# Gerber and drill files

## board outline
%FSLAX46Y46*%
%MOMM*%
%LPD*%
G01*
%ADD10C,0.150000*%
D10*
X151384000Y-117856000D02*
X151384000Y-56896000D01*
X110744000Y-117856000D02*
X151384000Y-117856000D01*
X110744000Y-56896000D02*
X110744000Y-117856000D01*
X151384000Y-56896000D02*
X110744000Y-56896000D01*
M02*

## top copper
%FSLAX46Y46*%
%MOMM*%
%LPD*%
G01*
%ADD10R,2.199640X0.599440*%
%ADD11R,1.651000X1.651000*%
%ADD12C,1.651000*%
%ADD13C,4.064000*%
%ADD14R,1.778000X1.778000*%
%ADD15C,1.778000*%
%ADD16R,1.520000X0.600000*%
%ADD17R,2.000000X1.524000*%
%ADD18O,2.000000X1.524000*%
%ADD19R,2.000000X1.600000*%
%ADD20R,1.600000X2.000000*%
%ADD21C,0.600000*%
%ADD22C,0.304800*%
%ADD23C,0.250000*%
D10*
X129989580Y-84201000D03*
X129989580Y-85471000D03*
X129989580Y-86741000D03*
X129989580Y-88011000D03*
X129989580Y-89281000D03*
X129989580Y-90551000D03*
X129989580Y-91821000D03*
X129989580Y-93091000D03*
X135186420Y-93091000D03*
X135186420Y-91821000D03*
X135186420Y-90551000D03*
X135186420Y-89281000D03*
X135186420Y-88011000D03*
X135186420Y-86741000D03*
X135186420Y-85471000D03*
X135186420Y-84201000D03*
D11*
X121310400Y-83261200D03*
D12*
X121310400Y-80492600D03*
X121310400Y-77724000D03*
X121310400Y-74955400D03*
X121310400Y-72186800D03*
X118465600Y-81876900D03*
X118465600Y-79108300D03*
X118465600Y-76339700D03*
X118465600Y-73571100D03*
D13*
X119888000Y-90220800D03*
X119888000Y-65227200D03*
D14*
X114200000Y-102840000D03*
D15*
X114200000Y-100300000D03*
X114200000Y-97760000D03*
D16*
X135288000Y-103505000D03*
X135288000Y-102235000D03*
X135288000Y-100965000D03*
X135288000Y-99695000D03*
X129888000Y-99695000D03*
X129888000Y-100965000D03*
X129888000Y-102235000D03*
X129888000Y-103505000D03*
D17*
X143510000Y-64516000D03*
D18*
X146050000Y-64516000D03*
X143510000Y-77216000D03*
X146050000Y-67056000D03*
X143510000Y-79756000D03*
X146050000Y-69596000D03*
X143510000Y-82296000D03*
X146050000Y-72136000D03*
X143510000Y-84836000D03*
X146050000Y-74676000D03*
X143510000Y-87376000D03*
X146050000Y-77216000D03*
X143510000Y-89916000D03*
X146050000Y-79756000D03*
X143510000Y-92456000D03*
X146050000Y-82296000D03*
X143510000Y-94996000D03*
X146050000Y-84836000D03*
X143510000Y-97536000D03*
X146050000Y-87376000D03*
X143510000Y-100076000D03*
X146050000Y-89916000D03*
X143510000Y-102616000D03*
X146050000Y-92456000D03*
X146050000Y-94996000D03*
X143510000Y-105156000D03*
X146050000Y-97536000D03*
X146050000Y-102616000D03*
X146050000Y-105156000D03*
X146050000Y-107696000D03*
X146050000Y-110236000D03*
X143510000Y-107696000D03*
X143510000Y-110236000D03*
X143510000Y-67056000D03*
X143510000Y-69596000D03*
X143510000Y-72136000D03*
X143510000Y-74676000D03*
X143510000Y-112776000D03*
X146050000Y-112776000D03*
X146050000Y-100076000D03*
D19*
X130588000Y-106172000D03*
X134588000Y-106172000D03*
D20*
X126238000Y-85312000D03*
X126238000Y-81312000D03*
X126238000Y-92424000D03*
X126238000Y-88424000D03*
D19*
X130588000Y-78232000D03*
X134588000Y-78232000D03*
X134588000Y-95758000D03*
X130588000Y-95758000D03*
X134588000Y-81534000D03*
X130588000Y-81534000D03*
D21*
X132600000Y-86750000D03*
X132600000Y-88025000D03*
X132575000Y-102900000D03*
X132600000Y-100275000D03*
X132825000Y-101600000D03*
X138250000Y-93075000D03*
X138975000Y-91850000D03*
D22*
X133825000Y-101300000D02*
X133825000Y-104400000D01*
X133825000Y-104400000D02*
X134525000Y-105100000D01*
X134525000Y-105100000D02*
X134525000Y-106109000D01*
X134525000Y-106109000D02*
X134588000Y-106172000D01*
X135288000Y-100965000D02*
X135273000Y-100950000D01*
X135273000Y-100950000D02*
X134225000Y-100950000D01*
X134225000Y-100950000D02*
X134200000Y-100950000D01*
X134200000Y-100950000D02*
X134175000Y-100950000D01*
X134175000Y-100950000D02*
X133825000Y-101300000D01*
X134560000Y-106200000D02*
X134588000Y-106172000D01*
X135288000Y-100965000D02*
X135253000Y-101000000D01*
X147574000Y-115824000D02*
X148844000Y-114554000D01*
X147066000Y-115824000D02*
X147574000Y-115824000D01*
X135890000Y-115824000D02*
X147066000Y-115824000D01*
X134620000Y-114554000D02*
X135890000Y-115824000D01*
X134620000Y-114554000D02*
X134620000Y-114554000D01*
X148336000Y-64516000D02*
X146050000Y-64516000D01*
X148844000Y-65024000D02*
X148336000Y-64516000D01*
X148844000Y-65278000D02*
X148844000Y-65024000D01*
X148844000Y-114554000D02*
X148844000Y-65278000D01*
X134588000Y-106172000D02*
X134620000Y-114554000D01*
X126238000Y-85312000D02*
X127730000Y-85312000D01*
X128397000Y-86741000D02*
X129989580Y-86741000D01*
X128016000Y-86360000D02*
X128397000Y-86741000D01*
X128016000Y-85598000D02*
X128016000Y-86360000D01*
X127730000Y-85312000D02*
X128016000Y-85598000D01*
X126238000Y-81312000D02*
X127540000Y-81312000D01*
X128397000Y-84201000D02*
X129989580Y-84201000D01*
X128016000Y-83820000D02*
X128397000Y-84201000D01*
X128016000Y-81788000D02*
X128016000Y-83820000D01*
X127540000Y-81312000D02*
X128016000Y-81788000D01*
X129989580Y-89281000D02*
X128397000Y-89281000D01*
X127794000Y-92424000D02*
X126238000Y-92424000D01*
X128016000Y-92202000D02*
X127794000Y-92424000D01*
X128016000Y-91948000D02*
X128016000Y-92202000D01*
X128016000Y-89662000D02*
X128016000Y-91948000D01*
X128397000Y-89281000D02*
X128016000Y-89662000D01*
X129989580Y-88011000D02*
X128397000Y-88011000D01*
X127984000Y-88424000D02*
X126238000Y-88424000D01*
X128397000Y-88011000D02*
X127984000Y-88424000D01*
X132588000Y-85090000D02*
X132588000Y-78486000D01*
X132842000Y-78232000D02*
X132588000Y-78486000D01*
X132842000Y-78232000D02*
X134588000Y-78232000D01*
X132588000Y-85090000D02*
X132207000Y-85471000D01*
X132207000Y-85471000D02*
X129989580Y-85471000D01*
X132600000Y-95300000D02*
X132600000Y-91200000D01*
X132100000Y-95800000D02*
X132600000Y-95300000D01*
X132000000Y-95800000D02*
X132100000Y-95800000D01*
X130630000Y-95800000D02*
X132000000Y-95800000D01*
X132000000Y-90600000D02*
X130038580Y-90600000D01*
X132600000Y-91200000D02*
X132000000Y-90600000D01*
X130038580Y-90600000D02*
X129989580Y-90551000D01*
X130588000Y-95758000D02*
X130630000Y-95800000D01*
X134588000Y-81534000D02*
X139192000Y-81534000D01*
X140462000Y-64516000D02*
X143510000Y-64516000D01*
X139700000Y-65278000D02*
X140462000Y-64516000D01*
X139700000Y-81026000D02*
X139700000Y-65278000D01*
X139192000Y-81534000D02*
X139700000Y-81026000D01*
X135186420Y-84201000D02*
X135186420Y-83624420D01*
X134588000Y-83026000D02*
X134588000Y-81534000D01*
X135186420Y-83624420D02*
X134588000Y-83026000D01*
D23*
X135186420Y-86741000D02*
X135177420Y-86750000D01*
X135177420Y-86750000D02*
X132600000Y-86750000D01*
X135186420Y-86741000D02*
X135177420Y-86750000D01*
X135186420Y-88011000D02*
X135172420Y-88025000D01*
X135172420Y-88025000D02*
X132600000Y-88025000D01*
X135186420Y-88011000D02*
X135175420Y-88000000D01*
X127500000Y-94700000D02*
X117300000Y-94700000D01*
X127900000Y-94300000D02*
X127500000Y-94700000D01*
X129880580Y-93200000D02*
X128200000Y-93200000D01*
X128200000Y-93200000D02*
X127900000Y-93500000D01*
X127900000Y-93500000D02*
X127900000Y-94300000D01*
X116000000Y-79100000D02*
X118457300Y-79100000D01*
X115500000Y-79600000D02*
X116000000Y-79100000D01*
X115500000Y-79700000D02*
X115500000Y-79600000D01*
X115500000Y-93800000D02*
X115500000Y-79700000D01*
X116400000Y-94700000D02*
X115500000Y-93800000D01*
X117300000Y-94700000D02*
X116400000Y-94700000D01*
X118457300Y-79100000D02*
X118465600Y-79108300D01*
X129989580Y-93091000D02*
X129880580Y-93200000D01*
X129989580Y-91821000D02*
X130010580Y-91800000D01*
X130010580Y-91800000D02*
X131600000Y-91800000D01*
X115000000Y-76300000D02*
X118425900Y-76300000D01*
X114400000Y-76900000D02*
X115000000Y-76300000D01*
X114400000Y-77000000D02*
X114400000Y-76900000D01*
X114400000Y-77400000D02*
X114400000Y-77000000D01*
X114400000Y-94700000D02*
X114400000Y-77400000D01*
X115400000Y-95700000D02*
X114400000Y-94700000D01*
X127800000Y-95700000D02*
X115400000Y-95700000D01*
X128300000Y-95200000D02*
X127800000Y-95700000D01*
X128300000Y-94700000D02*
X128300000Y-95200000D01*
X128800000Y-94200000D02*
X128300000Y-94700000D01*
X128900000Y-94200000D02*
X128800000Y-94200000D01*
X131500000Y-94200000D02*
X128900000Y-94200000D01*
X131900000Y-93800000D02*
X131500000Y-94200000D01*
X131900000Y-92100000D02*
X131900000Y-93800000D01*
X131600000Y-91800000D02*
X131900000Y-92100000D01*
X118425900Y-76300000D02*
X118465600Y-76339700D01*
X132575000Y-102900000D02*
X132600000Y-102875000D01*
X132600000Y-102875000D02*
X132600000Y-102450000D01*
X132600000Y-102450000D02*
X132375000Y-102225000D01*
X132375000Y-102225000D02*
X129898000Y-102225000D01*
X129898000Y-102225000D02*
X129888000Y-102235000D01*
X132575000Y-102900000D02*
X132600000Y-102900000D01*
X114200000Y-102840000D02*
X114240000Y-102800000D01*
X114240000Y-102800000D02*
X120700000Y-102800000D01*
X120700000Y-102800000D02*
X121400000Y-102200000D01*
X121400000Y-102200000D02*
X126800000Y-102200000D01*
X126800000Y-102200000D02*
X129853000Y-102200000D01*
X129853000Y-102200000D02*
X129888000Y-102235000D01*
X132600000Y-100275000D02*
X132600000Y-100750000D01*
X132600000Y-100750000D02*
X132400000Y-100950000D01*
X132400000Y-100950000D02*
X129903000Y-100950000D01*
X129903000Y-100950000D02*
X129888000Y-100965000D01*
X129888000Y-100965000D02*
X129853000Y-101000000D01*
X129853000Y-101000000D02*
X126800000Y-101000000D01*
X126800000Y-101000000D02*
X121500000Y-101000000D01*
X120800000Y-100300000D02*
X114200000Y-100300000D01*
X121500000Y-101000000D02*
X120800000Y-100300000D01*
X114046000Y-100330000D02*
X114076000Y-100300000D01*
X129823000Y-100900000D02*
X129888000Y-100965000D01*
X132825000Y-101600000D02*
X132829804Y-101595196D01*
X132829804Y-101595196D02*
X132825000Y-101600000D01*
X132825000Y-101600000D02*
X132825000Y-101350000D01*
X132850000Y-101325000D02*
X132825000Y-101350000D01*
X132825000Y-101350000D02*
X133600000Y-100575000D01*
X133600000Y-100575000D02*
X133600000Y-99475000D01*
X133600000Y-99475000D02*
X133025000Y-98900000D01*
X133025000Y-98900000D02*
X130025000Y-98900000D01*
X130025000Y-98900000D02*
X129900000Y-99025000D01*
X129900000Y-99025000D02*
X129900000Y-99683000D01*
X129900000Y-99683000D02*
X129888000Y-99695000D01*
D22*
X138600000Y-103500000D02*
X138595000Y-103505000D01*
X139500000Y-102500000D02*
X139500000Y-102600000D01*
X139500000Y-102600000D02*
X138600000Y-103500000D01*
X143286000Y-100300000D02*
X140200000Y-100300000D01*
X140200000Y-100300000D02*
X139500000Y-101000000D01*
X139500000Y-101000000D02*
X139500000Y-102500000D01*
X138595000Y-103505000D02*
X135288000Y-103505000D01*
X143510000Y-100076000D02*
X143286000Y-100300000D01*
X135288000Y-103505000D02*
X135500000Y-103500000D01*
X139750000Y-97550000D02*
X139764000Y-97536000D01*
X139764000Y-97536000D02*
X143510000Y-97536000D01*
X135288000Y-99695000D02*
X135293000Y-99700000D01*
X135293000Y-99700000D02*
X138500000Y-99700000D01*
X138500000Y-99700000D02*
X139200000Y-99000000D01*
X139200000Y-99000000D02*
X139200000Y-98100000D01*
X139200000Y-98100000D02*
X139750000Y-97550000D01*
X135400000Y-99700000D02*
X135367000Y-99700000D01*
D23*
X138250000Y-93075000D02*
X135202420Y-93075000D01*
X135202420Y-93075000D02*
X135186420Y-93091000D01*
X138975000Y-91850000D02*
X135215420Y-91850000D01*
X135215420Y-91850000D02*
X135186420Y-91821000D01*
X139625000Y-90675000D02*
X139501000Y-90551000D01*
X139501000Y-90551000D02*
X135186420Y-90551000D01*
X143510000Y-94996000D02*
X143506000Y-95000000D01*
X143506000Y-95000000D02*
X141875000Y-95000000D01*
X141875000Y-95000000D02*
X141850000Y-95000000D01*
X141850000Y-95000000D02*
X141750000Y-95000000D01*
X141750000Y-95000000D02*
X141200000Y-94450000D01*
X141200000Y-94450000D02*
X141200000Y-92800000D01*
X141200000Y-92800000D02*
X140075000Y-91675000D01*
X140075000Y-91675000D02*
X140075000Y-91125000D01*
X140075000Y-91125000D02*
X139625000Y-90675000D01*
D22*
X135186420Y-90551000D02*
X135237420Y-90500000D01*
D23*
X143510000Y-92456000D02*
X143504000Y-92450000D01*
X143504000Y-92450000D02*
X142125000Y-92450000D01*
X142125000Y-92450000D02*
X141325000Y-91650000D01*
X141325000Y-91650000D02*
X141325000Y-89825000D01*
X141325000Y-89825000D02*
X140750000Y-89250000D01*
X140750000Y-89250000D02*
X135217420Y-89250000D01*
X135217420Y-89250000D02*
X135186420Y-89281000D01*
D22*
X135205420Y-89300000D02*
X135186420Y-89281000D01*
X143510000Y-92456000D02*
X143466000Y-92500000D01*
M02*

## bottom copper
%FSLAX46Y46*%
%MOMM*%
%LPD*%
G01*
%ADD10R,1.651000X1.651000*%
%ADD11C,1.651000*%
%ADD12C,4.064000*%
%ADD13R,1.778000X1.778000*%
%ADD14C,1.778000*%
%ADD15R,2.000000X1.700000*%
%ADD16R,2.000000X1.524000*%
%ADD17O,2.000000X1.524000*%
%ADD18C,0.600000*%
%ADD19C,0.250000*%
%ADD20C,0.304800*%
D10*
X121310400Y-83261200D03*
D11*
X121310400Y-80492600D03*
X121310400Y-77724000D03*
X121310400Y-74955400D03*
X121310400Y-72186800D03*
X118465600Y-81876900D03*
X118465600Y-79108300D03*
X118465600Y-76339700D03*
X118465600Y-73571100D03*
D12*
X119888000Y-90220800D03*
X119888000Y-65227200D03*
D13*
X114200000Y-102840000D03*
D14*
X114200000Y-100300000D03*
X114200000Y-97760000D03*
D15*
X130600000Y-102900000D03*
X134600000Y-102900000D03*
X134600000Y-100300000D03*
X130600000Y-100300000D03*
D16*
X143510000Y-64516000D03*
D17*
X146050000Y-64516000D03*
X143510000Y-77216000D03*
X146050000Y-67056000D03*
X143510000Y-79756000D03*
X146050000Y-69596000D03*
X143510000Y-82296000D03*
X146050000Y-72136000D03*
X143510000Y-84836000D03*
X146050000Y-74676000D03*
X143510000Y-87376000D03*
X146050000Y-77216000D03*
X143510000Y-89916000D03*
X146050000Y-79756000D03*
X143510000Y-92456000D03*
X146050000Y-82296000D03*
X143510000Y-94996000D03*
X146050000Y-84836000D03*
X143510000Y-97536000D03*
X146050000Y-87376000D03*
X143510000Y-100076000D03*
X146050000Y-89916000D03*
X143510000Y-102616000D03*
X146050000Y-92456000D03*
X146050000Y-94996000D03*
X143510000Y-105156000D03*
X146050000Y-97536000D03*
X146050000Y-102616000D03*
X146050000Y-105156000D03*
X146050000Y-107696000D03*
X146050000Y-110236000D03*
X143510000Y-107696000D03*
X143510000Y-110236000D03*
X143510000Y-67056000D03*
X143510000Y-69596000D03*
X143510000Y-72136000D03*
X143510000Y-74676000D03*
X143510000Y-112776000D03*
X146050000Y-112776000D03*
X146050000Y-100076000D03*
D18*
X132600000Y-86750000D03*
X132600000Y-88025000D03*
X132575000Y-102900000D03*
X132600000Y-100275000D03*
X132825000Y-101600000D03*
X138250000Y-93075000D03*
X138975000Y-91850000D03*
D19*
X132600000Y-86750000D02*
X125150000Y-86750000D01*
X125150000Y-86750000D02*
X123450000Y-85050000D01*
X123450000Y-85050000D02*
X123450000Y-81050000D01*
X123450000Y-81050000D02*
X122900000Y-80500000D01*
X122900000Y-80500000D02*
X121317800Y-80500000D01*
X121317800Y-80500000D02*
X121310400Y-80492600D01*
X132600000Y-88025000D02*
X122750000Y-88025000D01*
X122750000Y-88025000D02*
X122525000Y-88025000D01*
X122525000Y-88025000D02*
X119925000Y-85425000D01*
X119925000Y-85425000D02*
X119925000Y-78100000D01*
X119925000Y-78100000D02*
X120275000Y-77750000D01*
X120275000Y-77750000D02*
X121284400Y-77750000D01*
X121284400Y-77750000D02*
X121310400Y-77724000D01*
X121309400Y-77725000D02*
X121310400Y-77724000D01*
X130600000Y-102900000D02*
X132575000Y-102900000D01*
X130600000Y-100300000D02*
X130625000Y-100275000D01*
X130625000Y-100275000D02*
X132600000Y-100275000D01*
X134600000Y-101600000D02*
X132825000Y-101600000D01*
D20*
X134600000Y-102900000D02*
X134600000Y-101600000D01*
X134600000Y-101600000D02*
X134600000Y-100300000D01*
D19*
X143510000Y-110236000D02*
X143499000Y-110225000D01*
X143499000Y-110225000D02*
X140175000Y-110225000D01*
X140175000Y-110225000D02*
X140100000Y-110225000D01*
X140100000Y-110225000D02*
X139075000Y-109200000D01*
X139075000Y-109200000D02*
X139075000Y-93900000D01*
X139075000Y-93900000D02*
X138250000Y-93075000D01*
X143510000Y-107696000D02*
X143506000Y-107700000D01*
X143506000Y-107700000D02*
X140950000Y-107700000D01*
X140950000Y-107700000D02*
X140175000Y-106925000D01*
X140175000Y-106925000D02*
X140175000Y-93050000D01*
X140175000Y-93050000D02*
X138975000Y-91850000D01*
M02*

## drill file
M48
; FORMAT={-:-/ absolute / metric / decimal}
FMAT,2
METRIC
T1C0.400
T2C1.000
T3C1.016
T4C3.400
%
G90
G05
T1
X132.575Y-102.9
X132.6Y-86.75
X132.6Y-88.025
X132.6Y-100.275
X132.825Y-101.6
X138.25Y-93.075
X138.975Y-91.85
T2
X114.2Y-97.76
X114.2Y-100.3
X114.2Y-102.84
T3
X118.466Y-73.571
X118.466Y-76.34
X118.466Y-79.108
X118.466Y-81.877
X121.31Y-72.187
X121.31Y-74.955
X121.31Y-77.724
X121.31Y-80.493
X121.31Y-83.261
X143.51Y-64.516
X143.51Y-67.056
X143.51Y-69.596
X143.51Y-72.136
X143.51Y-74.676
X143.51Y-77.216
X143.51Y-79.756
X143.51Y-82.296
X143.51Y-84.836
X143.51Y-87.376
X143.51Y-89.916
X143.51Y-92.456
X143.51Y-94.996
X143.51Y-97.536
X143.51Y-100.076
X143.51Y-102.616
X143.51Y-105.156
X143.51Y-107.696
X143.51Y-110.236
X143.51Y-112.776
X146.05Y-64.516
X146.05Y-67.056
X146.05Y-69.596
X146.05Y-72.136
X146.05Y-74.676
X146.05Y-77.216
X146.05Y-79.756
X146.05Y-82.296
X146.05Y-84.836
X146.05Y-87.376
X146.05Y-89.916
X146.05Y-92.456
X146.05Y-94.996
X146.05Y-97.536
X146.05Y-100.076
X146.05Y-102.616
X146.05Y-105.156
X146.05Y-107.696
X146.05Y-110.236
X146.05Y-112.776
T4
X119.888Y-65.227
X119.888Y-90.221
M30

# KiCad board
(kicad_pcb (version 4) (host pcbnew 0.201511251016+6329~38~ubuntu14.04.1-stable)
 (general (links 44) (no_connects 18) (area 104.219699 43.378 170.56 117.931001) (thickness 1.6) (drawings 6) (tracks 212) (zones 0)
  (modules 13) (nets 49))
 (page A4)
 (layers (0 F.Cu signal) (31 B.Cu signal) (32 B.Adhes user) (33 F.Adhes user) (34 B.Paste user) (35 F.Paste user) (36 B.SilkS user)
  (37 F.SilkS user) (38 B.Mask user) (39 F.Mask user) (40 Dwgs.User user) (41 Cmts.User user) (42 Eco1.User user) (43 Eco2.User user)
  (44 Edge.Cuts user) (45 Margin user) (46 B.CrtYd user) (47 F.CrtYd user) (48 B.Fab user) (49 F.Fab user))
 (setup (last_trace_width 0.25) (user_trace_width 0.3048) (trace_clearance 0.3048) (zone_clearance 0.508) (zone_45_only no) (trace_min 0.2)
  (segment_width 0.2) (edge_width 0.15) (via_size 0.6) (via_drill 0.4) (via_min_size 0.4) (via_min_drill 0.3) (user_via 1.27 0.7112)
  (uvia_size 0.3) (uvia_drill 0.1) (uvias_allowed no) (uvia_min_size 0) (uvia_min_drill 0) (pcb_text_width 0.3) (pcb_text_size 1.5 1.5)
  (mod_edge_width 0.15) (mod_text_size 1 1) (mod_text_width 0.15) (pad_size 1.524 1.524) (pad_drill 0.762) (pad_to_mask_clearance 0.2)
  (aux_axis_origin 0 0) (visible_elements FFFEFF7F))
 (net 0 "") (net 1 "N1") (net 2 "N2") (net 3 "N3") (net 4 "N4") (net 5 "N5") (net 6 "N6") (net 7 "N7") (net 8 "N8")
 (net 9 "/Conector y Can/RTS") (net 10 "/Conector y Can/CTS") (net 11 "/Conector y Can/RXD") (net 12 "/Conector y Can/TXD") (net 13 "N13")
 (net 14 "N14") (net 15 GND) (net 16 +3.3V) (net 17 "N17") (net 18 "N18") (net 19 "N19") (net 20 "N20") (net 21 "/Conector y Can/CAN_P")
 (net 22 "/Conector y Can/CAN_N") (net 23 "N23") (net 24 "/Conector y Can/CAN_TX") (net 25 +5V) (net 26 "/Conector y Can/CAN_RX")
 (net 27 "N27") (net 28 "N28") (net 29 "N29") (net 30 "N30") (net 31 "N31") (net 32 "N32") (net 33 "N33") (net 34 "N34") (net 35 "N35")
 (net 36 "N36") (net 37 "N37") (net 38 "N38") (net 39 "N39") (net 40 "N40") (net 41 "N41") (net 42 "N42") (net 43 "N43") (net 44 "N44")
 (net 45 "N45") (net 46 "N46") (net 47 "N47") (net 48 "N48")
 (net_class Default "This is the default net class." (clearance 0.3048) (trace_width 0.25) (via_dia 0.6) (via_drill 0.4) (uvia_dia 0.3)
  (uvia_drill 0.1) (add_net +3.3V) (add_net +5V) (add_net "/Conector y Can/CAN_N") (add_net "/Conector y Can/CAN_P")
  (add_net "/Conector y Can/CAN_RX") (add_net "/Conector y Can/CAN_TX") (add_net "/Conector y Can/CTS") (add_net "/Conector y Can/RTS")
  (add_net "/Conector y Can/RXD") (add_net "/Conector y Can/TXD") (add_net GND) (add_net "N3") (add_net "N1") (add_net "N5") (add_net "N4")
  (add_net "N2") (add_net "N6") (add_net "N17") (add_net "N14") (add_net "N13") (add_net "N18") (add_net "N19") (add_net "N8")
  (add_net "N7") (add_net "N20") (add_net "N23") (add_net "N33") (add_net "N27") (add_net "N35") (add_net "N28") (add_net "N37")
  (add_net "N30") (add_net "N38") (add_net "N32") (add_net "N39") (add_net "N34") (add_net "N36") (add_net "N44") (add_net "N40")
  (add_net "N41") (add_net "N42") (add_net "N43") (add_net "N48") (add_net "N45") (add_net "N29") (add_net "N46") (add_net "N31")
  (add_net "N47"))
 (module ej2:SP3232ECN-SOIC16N (layer F.Cu) (at 132.588 88.646 270)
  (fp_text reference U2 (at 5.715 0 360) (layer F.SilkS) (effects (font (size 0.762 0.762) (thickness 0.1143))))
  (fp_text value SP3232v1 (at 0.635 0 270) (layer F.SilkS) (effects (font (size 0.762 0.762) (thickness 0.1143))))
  (pad 1 smd rect (at -4.445 2.59842 270) (size 0.59944 2.19964) (layers F.Cu F.Paste F.Mask) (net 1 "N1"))
  (pad 2 smd rect (at -3.175 2.59842 270) (size 0.59944 2.19964) (layers F.Cu F.Paste F.Mask) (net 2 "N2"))
  (pad 3 smd rect (at -1.905 2.59842 270) (size 0.59944 2.19964) (layers F.Cu F.Paste F.Mask) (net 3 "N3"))
  (pad 4 smd rect (at -0.635 2.59842 270) (size 0.59944 2.19964) (layers F.Cu F.Paste F.Mask) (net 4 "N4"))
  (pad 5 smd rect (at 0.635 2.59842 270) (size 0.59944 2.19964) (layers F.Cu F.Paste F.Mask) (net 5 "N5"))
  (pad 6 smd rect (at 1.905 2.59842 270) (size 0.59944 2.19964) (layers F.Cu F.Paste F.Mask) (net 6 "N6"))
  (pad 7 smd rect (at 3.175 2.59842 270) (size 0.59944 2.19964) (layers F.Cu F.Paste F.Mask) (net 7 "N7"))
  (pad 8 smd rect (at 4.445 2.59842 270) (size 0.59944 2.19964) (layers F.Cu F.Paste F.Mask) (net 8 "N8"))
  (pad 9 smd rect (at 4.445 -2.59842 270) (size 0.59944 2.19964) (layers F.Cu F.Paste F.Mask) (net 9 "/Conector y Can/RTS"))
  (pad 10 smd rect (at 3.175 -2.59842 270) (size 0.59944 2.19964) (layers F.Cu F.Paste F.Mask) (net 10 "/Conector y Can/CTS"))
  (pad 11 smd rect (at 1.905 -2.59842 270) (size 0.59944 2.19964) (layers F.Cu F.Paste F.Mask) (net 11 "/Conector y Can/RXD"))
  (pad 12 smd rect (at 0.635 -2.59842 270) (size 0.59944 2.19964) (layers F.Cu F.Paste F.Mask) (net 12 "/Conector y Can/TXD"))
  (pad 13 smd rect (at -0.635 -2.59842 270) (size 0.59944 2.19964) (layers F.Cu F.Paste F.Mask) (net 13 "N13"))
  (pad 14 smd rect (at -1.905 -2.59842 270) (size 0.59944 2.19964) (layers F.Cu F.Paste F.Mask) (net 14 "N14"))
  (pad 15 smd rect (at -3.175 -2.59842 270) (size 0.59944 2.19964) (layers F.Cu F.Paste F.Mask) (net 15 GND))
  (pad 16 smd rect (at -4.445 -2.59842 270) (size 0.59944 2.19964) (layers F.Cu F.Paste F.Mask) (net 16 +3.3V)))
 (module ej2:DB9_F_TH (layer F.Cu) (at 119.888 77.724 90)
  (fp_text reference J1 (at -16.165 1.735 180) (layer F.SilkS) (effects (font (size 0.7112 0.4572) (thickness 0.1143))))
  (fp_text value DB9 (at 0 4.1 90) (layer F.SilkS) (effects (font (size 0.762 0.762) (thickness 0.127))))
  (pad 1 thru_hole rect (at -5.5372 1.4224 90) (size 1.651 1.651) (drill 1.016) (layers *.Cu *.Mask) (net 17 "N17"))
  (pad 2 thru_hole circle (at -2.7686 1.4224 90) (size 1.651 1.651) (drill 1.016) (layers *.Cu *.Mask) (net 14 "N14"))
  (pad 3 thru_hole circle (at 0 1.4224 90) (size 1.651 1.651) (drill 1.016) (layers *.Cu *.Mask) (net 13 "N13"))
  (pad 4 thru_hole circle (at 2.7686 1.4224 90) (size 1.651 1.651) (drill 1.016) (layers *.Cu *.Mask) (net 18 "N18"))
  (pad 5 thru_hole circle (at 5.5372 1.4224 90) (size 1.651 1.651) (drill 1.016) (layers *.Cu *.Mask) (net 15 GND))
  (pad 6 thru_hole circle (at -4.1529 -1.4224 90) (size 1.651 1.651) (drill 1.016) (layers *.Cu *.Mask) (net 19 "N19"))
  (pad 7 thru_hole circle (at -1.3843 -1.4224 90) (size 1.651 1.651) (drill 1.016) (layers *.Cu *.Mask) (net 8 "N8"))
  (pad 8 thru_hole circle (at 1.3843 -1.4224 90) (size 1.651 1.651) (drill 1.016) (layers *.Cu *.Mask) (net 7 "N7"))
  (pad 9 thru_hole circle (at 4.1529 -1.4224 90) (size 1.651 1.651) (drill 1.016) (layers *.Cu *.Mask) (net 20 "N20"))
  (pad 10 thru_hole circle (at -12.4968 0 90) (size 4.064 4.064) (drill 3.4) (layers *.Cu *.Mask))
  (pad 11 thru_hole circle (at 12.4968 0 90) (size 4.064 4.064) (drill 3.4) (layers *.Cu *.Mask)))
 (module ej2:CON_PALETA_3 (layer F.Cu) (at 114.2 100.3 90)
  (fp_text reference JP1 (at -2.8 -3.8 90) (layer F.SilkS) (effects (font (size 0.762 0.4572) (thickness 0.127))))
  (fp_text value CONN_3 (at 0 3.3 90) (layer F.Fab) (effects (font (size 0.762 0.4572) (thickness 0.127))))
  (pad 1 thru_hole rect (at -2.54 0 90) (size 1.778 1.778) (drill 1) (layers *.Cu *.Mask) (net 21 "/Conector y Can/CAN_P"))
  (pad 2 thru_hole circle (at 0 0 90) (size 1.778 1.778) (drill 1) (layers *.Cu *.Mask) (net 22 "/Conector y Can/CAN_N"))
  (pad 3 thru_hole circle (at 2.54 0 90) (size 1.778 1.778) (drill 1) (layers *.Cu *.Mask) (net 15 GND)))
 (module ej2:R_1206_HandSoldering (layer B.Cu) (at 132.6 102.9)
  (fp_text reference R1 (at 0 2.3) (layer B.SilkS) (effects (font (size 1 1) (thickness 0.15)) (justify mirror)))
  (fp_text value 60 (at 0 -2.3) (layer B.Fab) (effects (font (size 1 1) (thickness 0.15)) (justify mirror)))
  (pad 1 smd rect (at -2 0) (size 2 1.7) (layers B.Cu B.Paste B.Mask) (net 21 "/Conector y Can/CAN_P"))
  (pad 2 smd rect (at 2 0) (size 2 1.7) (layers B.Cu B.Paste B.Mask) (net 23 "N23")))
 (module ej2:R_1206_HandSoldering (layer B.Cu) (at 132.6 100.3 180)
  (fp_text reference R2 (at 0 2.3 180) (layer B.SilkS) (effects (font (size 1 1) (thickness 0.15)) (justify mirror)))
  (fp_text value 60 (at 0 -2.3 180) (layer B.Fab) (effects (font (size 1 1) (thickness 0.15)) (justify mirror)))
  (pad 1 smd rect (at -2 0 180) (size 2 1.7) (layers B.Cu B.Paste B.Mask) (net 23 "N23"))
  (pad 2 smd rect (at 2 0 180) (size 2 1.7) (layers B.Cu B.Paste B.Mask) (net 22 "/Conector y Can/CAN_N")))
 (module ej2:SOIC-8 (layer F.Cu) (at 132.588 101.6 180)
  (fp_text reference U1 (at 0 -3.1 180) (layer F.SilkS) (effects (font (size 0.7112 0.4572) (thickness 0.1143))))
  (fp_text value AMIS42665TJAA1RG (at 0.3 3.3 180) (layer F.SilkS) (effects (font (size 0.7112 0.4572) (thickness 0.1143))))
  (pad 1 smd rect (at -2.7 -1.905 90) (size 0.6 1.52) (layers F.Cu F.Paste F.Mask) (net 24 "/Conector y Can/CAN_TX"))
  (pad 2 smd rect (at -2.7 -0.635 90) (size 0.6 1.52) (layers F.Cu F.Paste F.Mask) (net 15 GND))
  (pad 3 smd rect (at -2.7 0.635 90) (size 0.6 1.52) (layers F.Cu F.Paste F.Mask) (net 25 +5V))
  (pad 4 smd rect (at -2.7 1.905 90) (size 0.6 1.52) (layers F.Cu F.Paste F.Mask) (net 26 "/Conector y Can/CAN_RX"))
  (pad 5 smd rect (at 2.7 1.905 90) (size 0.6 1.52) (layers F.Cu F.Paste F.Mask) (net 23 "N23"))
  (pad 6 smd rect (at 2.7 0.635 90) (size 0.6 1.52) (layers F.Cu F.Paste F.Mask) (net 22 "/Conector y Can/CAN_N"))
  (pad 7 smd rect (at 2.7 -0.635 90) (size 0.6 1.52) (layers F.Cu F.Paste F.Mask) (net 21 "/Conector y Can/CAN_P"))
  (pad 8 smd rect (at 2.7 -1.905 90) (size 0.6 1.52) (layers F.Cu F.Paste F.Mask) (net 15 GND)))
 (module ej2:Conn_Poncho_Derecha (layer F.Cu) (at 143.51 64.516)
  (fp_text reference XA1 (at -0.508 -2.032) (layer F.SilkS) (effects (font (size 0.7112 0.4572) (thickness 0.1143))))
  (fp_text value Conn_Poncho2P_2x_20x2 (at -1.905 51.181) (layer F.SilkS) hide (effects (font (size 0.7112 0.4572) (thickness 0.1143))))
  (pad 1 thru_hole rect (at 0 0 270) (size 1.524 2) (drill 1.016) (layers *.Cu *.Mask) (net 16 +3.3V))
  (pad 2 thru_hole oval (at 2.54 0 270) (size 1.524 2) (drill 1.016) (layers *.Cu *.Mask) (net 25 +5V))
  (pad 11 thru_hole oval (at 0 12.7 270) (size 1.524 2) (drill 1.016) (layers *.Cu *.Mask) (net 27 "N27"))
  (pad 4 thru_hole oval (at 2.54 2.54 270) (size 1.524 2) (drill 1.016) (layers *.Cu *.Mask) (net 15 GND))
  (pad 13 thru_hole oval (at 0 15.24 270) (size 1.524 2) (drill 1.016) (layers *.Cu *.Mask) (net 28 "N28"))
  (pad 6 thru_hole oval (at 2.54 5.08 270) (size 1.524 2) (drill 1.016) (layers *.Cu *.Mask) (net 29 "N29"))
  (pad 15 thru_hole oval (at 0 17.78 270) (size 1.524 2) (drill 1.016) (layers *.Cu *.Mask) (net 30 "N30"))
  (pad 8 thru_hole oval (at 2.54 7.62 270) (size 1.524 2) (drill 1.016) (layers *.Cu *.Mask) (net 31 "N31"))
  (pad 17 thru_hole oval (at 0 20.32 270) (size 1.524 2) (drill 1.016) (layers *.Cu *.Mask) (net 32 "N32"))
  (pad 10 thru_hole oval (at 2.54 10.16 270) (size 1.524 2) (drill 1.016) (layers *.Cu *.Mask) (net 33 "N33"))
  (pad 19 thru_hole oval (at 0 22.86 270) (size 1.524 2) (drill 1.016) (layers *.Cu *.Mask) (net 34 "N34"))
  (pad 12 thru_hole oval (at 2.54 12.7 270) (size 1.524 2) (drill 1.016) (layers *.Cu *.Mask) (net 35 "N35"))
  (pad 21 thru_hole oval (at 0 25.4 270) (size 1.524 2) (drill 1.016) (layers *.Cu *.Mask) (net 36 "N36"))
  (pad 14 thru_hole oval (at 2.54 15.24 270) (size 1.524 2) (drill 1.016) (layers *.Cu *.Mask) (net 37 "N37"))
  (pad 23 thru_hole oval (at 0 27.94 270) (size 1.524 2) (drill 1.016) (layers *.Cu *.Mask) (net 12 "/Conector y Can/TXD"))
  (pad 16 thru_hole oval (at 2.54 17.78 270) (size 1.524 2) (drill 1.016) (layers *.Cu *.Mask) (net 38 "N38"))
  (pad 25 thru_hole oval (at 0 30.48 270) (size 1.524 2) (drill 1.016) (layers *.Cu *.Mask) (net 11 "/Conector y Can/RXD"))
  (pad 18 thru_hole oval (at 2.54 20.32 270) (size 1.524 2) (drill 1.016) (layers *.Cu *.Mask) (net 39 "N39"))
  (pad 27 thru_hole oval (at 0 33.02 270) (size 1.524 2) (drill 1.016) (layers *.Cu *.Mask) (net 26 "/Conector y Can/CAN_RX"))
  (pad 20 thru_hole oval (at 2.54 22.86 270) (size 1.524 2) (drill 1.016) (layers *.Cu *.Mask) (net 15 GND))
  (pad 29 thru_hole oval (at 0 35.56 270) (size 1.524 2) (drill 1.016) (layers *.Cu *.Mask) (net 24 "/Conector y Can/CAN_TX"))
  (pad 22 thru_hole oval (at 2.54 25.4 270) (size 1.524 2) (drill 1.016) (layers *.Cu *.Mask) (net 15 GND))
  (pad 31 thru_hole oval (at 0 38.1 270) (size 1.524 2) (drill 1.016) (layers *.Cu *.Mask) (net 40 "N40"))
  (pad 24 thru_hole oval (at 2.54 27.94 270) (size 1.524 2) (drill 1.016) (layers *.Cu *.Mask) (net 15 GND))
  (pad 26 thru_hole oval (at 2.54 30.48 270) (size 1.524 2) (drill 1.016) (layers *.Cu *.Mask) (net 15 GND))
  (pad 33 thru_hole oval (at 0 40.64 270) (size 1.524 2) (drill 1.016) (layers *.Cu *.Mask) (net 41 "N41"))
  (pad 28 thru_hole oval (at 2.54 33.02 270) (size 1.524 2) (drill 1.016) (layers *.Cu *.Mask) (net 15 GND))
  (pad 32 thru_hole oval (at 2.54 38.1 270) (size 1.524 2) (drill 1.016) (layers *.Cu *.Mask) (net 15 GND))
  (pad 34 thru_hole oval (at 2.54 40.64 270) (size 1.524 2) (drill 1.016) (layers *.Cu *.Mask) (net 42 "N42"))
  (pad 36 thru_hole oval (at 2.54 43.18 270) (size 1.524 2) (drill 1.016) (layers *.Cu *.Mask) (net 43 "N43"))
  (pad 38 thru_hole oval (at 2.54 45.72 270) (size 1.524 2) (drill 1.016) (layers *.Cu *.Mask) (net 15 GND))
  (pad 35 thru_hole oval (at 0 43.18 270) (size 1.524 2) (drill 1.016) (layers *.Cu *.Mask) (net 10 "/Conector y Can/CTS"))
  (pad 37 thru_hole oval (at 0 45.72 270) (size 1.524 2) (drill 1.016) (layers *.Cu *.Mask) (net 9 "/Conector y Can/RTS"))
  (pad 3 thru_hole oval (at 0 2.54 270) (size 1.524 2) (drill 1.016) (layers *.Cu *.Mask) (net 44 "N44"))
  (pad 5 thru_hole oval (at 0 5.08 270) (size 1.524 2) (drill 1.016) (layers *.Cu *.Mask) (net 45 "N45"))
  (pad 7 thru_hole oval (at 0 7.62 270) (size 1.524 2) (drill 1.016) (layers *.Cu *.Mask) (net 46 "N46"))
  (pad 9 thru_hole oval (at 0 10.16 270) (size 1.524 2) (drill 1.016) (layers *.Cu *.Mask) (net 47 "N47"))
  (pad 39 thru_hole oval (at 0 48.26 270) (size 1.524 2) (drill 1.016) (layers *.Cu *.Mask) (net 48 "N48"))
  (pad 40 thru_hole oval (at 2.54 48.26 270) (size 1.524 2) (drill 1.016) (layers *.Cu *.Mask) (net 15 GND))
  (pad 30 thru_hole oval (at 2.54 35.56 270) (size 1.524 2) (drill 1.016) (layers *.Cu *.Mask) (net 15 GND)))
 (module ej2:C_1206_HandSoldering (layer F.Cu) (at 132.588 106.172)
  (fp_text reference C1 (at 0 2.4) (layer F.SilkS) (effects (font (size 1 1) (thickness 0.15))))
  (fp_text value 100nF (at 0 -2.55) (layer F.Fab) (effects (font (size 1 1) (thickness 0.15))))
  (pad 1 smd rect (at -2 0) (size 2 1.6) (layers F.Cu F.Paste F.Mask) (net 15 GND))
  (pad 2 smd rect (at 2 0) (size 2 1.6) (layers F.Cu F.Paste F.Mask) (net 25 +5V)))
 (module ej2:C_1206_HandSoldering (layer F.Cu) (at 126.238 83.312 90)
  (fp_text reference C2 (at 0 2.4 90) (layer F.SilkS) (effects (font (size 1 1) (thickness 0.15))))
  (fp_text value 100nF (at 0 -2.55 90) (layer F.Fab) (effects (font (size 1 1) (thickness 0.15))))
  (pad 1 smd rect (at -2 0 90) (size 2 1.6) (layers F.Cu F.Paste F.Mask) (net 3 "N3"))
  (pad 2 smd rect (at 2 0 90) (size 2 1.6) (layers F.Cu F.Paste F.Mask) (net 1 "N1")))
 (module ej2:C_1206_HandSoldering (layer F.Cu) (at 126.238 90.424 90)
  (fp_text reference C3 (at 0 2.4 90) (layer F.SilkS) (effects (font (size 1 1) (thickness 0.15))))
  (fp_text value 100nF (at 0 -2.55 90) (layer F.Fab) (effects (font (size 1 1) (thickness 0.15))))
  (pad 1 smd rect (at -2 0 90) (size 2 1.6) (layers F.Cu F.Paste F.Mask) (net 5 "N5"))
  (pad 2 smd rect (at 2 0 90) (size 2 1.6) (layers F.Cu F.Paste F.Mask) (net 4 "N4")))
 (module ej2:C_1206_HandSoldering (layer F.Cu) (at 132.588 78.232)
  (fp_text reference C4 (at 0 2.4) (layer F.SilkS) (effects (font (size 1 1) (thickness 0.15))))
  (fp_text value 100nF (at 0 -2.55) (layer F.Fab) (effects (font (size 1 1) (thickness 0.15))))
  (pad 1 smd rect (at -2 0) (size 2 1.6) (layers F.Cu F.Paste F.Mask) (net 15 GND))
  (pad 2 smd rect (at 2 0) (size 2 1.6) (layers F.Cu F.Paste F.Mask) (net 2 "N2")))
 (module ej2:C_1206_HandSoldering (layer F.Cu) (at 132.588 95.758 180)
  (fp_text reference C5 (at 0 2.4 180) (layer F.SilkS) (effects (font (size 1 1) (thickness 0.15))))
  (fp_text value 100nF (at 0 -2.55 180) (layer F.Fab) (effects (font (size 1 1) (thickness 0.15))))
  (pad 1 smd rect (at -2 0 180) (size 2 1.6) (layers F.Cu F.Paste F.Mask) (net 15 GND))
  (pad 2 smd rect (at 2 0 180) (size 2 1.6) (layers F.Cu F.Paste F.Mask) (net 6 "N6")))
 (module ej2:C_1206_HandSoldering (layer F.Cu) (at 132.588 81.534 180)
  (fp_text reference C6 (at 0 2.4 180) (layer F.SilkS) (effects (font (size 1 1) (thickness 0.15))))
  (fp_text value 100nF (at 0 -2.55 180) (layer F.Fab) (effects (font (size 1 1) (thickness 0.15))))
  (pad 1 smd rect (at -2 0 180) (size 2 1.6) (layers F.Cu F.Paste F.Mask) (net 16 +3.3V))
  (pad 2 smd rect (at 2 0 180) (size 2 1.6) (layers F.Cu F.Paste F.Mask) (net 15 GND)))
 (gr_line (start 151.384 117.856) (end 151.384 56.896) (angle 90) (layer Edge.Cuts) (width 0.15))
 (gr_line (start 110.744 117.856) (end 151.384 117.856) (angle 90) (layer Edge.Cuts) (width 0.15))
 (gr_line (start 110.744 56.896) (end 110.744 117.856) (angle 90) (layer Edge.Cuts) (width 0.15))
 (gr_line (start 151.384 56.896) (end 110.744 56.896) (angle 90) (layer Edge.Cuts) (width 0.15))
 (segment (start 133.825 101.3) (end 133.825 104.4) (width 0.3048) (layer F.Cu) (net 25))
 (segment (start 133.825 104.4) (end 134.525 105.1) (width 0.3048) (layer F.Cu) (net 25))
 (segment (start 134.525 105.1) (end 134.525 106.109) (width 0.3048) (layer F.Cu) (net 25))
 (segment (start 134.525 106.109) (end 134.588 106.172) (width 0.3048) (layer F.Cu) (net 25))
 (segment (start 135.288 100.965) (end 135.273 100.95) (width 0.3048) (layer F.Cu) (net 25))
 (segment (start 135.273 100.95) (end 134.225 100.95) (width 0.3048) (layer F.Cu) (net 25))
 (segment (start 134.225 100.95) (end 134.2 100.95) (width 0.3048) (layer F.Cu) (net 25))
 (segment (start 134.2 100.95) (end 134.175 100.95) (width 0.3048) (layer F.Cu) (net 25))
 (segment (start 134.175 100.95) (end 133.825 101.3) (width 0.3048) (layer F.Cu) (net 25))
 (segment (start 134.56 106.2) (end 134.588 106.172) (width 0.3048) (layer F.Cu) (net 25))
 (segment (start 135.288 100.965) (end 135.253 101) (width 0.3048) (layer F.Cu) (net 25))
 (segment (start 147.574 115.824) (end 148.844 114.554) (width 0.3048) (layer F.Cu) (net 25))
 (segment (start 147.066 115.824) (end 147.574 115.824) (width 0.3048) (layer F.Cu) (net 25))
 (segment (start 135.89 115.824) (end 147.066 115.824) (width 0.3048) (layer F.Cu) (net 25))
 (segment (start 134.62 114.554) (end 135.89 115.824) (width 0.3048) (layer F.Cu) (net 25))
 (segment (start 134.62 114.554) (end 134.62 114.554) (width 0.3048) (layer F.Cu) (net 25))
 (segment (start 148.336 64.516) (end 146.05 64.516) (width 0.3048) (layer F.Cu) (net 25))
 (segment (start 148.844 65.024) (end 148.336 64.516) (width 0.3048) (layer F.Cu) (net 25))
 (segment (start 148.844 65.278) (end 148.844 65.024) (width 0.3048) (layer F.Cu) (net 25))
 (segment (start 148.844 114.554) (end 148.844 65.278) (width 0.3048) (layer F.Cu) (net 25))
 (segment (start 134.588 106.172) (end 134.62 114.554) (width 0.3048) (layer F.Cu) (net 25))
 (segment (start 126.238 85.312) (end 127.73 85.312) (width 0.3048) (layer F.Cu) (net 3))
 (segment (start 128.397 86.741) (end 129.98958 86.741) (width 0.3048) (layer F.Cu) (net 3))
 (segment (start 128.016 86.36) (end 128.397 86.741) (width 0.3048) (layer F.Cu) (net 3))
 (segment (start 128.016 85.598) (end 128.016 86.36) (width 0.3048) (layer F.Cu) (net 3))
 (segment (start 127.73 85.312) (end 128.016 85.598) (width 0.3048) (layer F.Cu) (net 3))
 (segment (start 126.238 81.312) (end 127.54 81.312) (width 0.3048) (layer F.Cu) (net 1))
 (segment (start 128.397 84.201) (end 129.98958 84.201) (width 0.3048) (layer F.Cu) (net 1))
 (segment (start 128.016 83.82) (end 128.397 84.201) (width 0.3048) (layer F.Cu) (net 1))
 (segment (start 128.016 81.788) (end 128.016 83.82) (width 0.3048) (layer F.Cu) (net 1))
 (segment (start 127.54 81.312) (end 128.016 81.788) (width 0.3048) (layer F.Cu) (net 1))
 (segment (start 129.98958 89.281) (end 128.397 89.281) (width 0.3048) (layer F.Cu) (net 5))
 (segment (start 127.794 92.424) (end 126.238 92.424) (width 0.3048) (layer F.Cu) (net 5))
 (segment (start 128.016 92.202) (end 127.794 92.424) (width 0.3048) (layer F.Cu) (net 5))
 (segment (start 128.016 91.948) (end 128.016 92.202) (width 0.3048) (layer F.Cu) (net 5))
 (segment (start 128.016 89.662) (end 128.016 91.948) (width 0.3048) (layer F.Cu) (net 5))
 (segment (start 128.397 89.281) (end 128.016 89.662) (width 0.3048) (layer F.Cu) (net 5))
 (segment (start 129.98958 88.011) (end 128.397 88.011) (width 0.3048) (layer F.Cu) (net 4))
 (segment (start 127.984 88.424) (end 126.238 88.424) (width 0.3048) (layer F.Cu) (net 4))
 (segment (start 128.397 88.011) (end 127.984 88.424) (width 0.3048) (layer F.Cu) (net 4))
 (segment (start 132.588 85.09) (end 132.588 78.486) (width 0.3048) (layer F.Cu) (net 2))
 (segment (start 132.842 78.232) (end 132.588 78.486) (width 0.3048) (layer F.Cu) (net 2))
 (segment (start 132.842 78.232) (end 134.588 78.232) (width 0.3048) (layer F.Cu) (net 2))
 (segment (start 132.588 85.09) (end 132.207 85.471) (width 0.3048) (layer F.Cu) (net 2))
 (segment (start 132.207 85.471) (end 129.98958 85.471) (width 0.3048) (layer F.Cu) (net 2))
 (segment (start 132.6 95.3) (end 132.6 91.2) (width 0.3048) (layer F.Cu) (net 6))
 (segment (start 132.1 95.8) (end 132.6 95.3) (width 0.3048) (layer F.Cu) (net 6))
 (segment (start 132 95.8) (end 132.1 95.8) (width 0.3048) (layer F.Cu) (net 6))
 (segment (start 130.63 95.8) (end 132 95.8) (width 0.3048) (layer F.Cu) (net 6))
 (segment (start 132 90.6) (end 130.03858 90.6) (width 0.3048) (layer F.Cu) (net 6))
 (segment (start 132.6 91.2) (end 132 90.6) (width 0.3048) (layer F.Cu) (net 6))
 (segment (start 130.03858 90.6) (end 129.98958 90.551) (width 0.3048) (layer F.Cu) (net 6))
 (segment (start 130.588 95.758) (end 130.63 95.8) (width 0.3048) (layer F.Cu) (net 6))
 (segment (start 134.588 81.534) (end 139.192 81.534) (width 0.3048) (layer F.Cu) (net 16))
 (segment (start 140.462 64.516) (end 143.51 64.516) (width 0.3048) (layer F.Cu) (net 16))
 (segment (start 139.7 65.278) (end 140.462 64.516) (width 0.3048) (layer F.Cu) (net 16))
 (segment (start 139.7 81.026) (end 139.7 65.278) (width 0.3048) (layer F.Cu) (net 16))
 (segment (start 139.192 81.534) (end 139.7 81.026) (width 0.3048) (layer F.Cu) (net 16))
 (segment (start 135.18642 84.201) (end 135.18642 83.62442) (width 0.3048) (layer F.Cu) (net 16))
 (segment (start 134.588 83.026) (end 134.588 81.534) (width 0.3048) (layer F.Cu) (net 16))
 (segment (start 135.18642 83.62442) (end 134.588 83.026) (width 0.3048) (layer F.Cu) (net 16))
 (segment (start 135.18642 86.741) (end 135.17742 86.75) (width 0.25) (layer F.Cu) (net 14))
 (segment (start 135.17742 86.75) (end 132.6 86.75) (width 0.25) (layer F.Cu) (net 14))
 (via (at 132.6 86.75) (size 0.6) (drill 0.4) (layers F.Cu B.Cu) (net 14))
 (segment (start 132.6 86.75) (end 125.15 86.75) (width 0.25) (layer B.Cu) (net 14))
 (segment (start 125.15 86.75) (end 123.45 85.05) (width 0.25) (layer B.Cu) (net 14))
 (segment (start 123.45 85.05) (end 123.45 81.05) (width 0.25) (layer B.Cu) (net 14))
 (segment (start 123.45 81.05) (end 122.9 80.5) (width 0.25) (layer B.Cu) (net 14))
 (segment (start 122.9 80.5) (end 121.3178 80.5) (width 0.25) (layer B.Cu) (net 14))
 (segment (start 121.3178 80.5) (end 121.3104 80.4926) (width 0.25) (layer B.Cu) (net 14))
 (segment (start 135.18642 86.741) (end 135.17742 86.75) (width 0.25) (layer F.Cu) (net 14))
 (segment (start 135.18642 88.011) (end 135.17242 88.025) (width 0.25) (layer F.Cu) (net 13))
 (segment (start 135.17242 88.025) (end 132.6 88.025) (width 0.25) (layer F.Cu) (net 13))
 (via (at 132.6 88.025) (size 0.6) (drill 0.4) (layers F.Cu B.Cu) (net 13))
 (segment (start 132.6 88.025) (end 122.75 88.025) (width 0.25) (layer B.Cu) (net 13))
 (segment (start 122.75 88.025) (end 122.525 88.025) (width 0.25) (layer B.Cu) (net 13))
 (segment (start 122.525 88.025) (end 119.925 85.425) (width 0.25) (layer B.Cu) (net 13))
 (segment (start 119.925 85.425) (end 119.925 78.1) (width 0.25) (layer B.Cu) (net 13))
 (segment (start 119.925 78.1) (end 120.275 77.75) (width 0.25) (layer B.Cu) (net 13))
 (segment (start 120.275 77.75) (end 121.2844 77.75) (width 0.25) (layer B.Cu) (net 13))
 (segment (start 121.2844 77.75) (end 121.3104 77.724) (width 0.25) (layer B.Cu) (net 13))
 (segment (start 135.18642 88.011) (end 135.17542 88) (width 0.25) (layer F.Cu) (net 13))
 (segment (start 121.3094 77.725) (end 121.3104 77.724) (width 0.25) (layer B.Cu) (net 13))
 (segment (start 127.5 94.7) (end 117.3 94.7) (width 0.25) (layer F.Cu) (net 8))
 (segment (start 127.9 94.3) (end 127.5 94.7) (width 0.25) (layer F.Cu) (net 8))
 (segment (start 129.88058 93.2) (end 128.2 93.2) (width 0.25) (layer F.Cu) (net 8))
 (segment (start 128.2 93.2) (end 127.9 93.5) (width 0.25) (layer F.Cu) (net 8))
 (segment (start 127.9 93.5) (end 127.9 94.3) (width 0.25) (layer F.Cu) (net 8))
 (segment (start 116 79.1) (end 118.4573 79.1) (width 0.25) (layer F.Cu) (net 8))
 (segment (start 115.5 79.6) (end 116 79.1) (width 0.25) (layer F.Cu) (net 8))
 (segment (start 115.5 79.7) (end 115.5 79.6) (width 0.25) (layer F.Cu) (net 8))
 (segment (start 115.5 93.8) (end 115.5 79.7) (width 0.25) (layer F.Cu) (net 8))
 (segment (start 116.4 94.7) (end 115.5 93.8) (width 0.25) (layer F.Cu) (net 8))
 (segment (start 117.3 94.7) (end 116.4 94.7) (width 0.25) (layer F.Cu) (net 8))
 (segment (start 118.4573 79.1) (end 118.4656 79.1083) (width 0.25) (layer F.Cu) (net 8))
 (segment (start 129.98958 93.091) (end 129.88058 93.2) (width 0.25) (layer F.Cu) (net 8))
 (segment (start 129.98958 91.821) (end 130.01058 91.8) (width 0.25) (layer F.Cu) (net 7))
 (segment (start 130.01058 91.8) (end 131.6 91.8) (width 0.25) (layer F.Cu) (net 7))
 (segment (start 115 76.3) (end 118.4259 76.3) (width 0.25) (layer F.Cu) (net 7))
 (segment (start 114.4 76.9) (end 115 76.3) (width 0.25) (layer F.Cu) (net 7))
 (segment (start 114.4 77) (end 114.4 76.9) (width 0.25) (layer F.Cu) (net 7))
 (segment (start 114.4 77.4) (end 114.4 77) (width 0.25) (layer F.Cu) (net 7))
 (segment (start 114.4 94.7) (end 114.4 77.4) (width 0.25) (layer F.Cu) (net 7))
 (segment (start 115.4 95.7) (end 114.4 94.7) (width 0.25) (layer F.Cu) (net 7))
 (segment (start 127.8 95.7) (end 115.4 95.7) (width 0.25) (layer F.Cu) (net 7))
 (segment (start 128.3 95.2) (end 127.8 95.7) (width 0.25) (layer F.Cu) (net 7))
 (segment (start 128.3 94.7) (end 128.3 95.2) (width 0.25) (layer F.Cu) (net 7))
 (segment (start 128.8 94.2) (end 128.3 94.7) (width 0.25) (layer F.Cu) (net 7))
 (segment (start 128.9 94.2) (end 128.8 94.2) (width 0.25) (layer F.Cu) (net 7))
 (segment (start 131.5 94.2) (end 128.9 94.2) (width 0.25) (layer F.Cu) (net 7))
 (segment (start 131.9 93.8) (end 131.5 94.2) (width 0.25) (layer F.Cu) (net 7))
 (segment (start 131.9 92.1) (end 131.9 93.8) (width 0.25) (layer F.Cu) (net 7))
 (segment (start 131.6 91.8) (end 131.9 92.1) (width 0.25) (layer F.Cu) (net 7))
 (segment (start 118.4259 76.3) (end 118.4656 76.3397) (width 0.25) (layer F.Cu) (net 7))
 (segment (start 132.575 102.9) (end 132.6 102.875) (width 0.25) (layer F.Cu) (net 21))
 (segment (start 132.6 102.875) (end 132.6 102.45) (width 0.25) (layer F.Cu) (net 21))
 (segment (start 132.6 102.45) (end 132.375 102.225) (width 0.25) (layer F.Cu) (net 21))
 (segment (start 132.375 102.225) (end 129.898 102.225) (width 0.25) (layer F.Cu) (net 21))
 (segment (start 129.898 102.225) (end 129.888 102.235) (width 0.25) (layer F.Cu) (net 21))
 (segment (start 130.6 102.9) (end 132.575 102.9) (width 0.25) (layer B.Cu) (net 21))
 (via (at 132.575 102.9) (size 0.6) (drill 0.4) (layers F.Cu B.Cu) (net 21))
 (segment (start 132.575 102.9) (end 132.6 102.9) (width 0.25) (layer F.Cu) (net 21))
 (segment (start 114.2 102.84) (end 114.24 102.8) (width 0.25) (layer F.Cu) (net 21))
 (segment (start 114.24 102.8) (end 120.7 102.8) (width 0.25) (layer F.Cu) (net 21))
 (segment (start 120.7 102.8) (end 121.4 102.2) (width 0.25) (layer F.Cu) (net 21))
 (segment (start 121.4 102.2) (end 126.8 102.2) (width 0.25) (layer F.Cu) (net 21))
 (segment (start 126.8 102.2) (end 129.853 102.2) (width 0.25) (layer F.Cu) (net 21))
 (segment (start 129.853 102.2) (end 129.888 102.235) (width 0.25) (layer F.Cu) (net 21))
 (segment (start 130.6 100.3) (end 130.625 100.275) (width 0.25) (layer B.Cu) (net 22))
 (segment (start 130.625 100.275) (end 132.6 100.275) (width 0.25) (layer B.Cu) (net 22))
 (via (at 132.6 100.275) (size 0.6) (drill 0.4) (layers F.Cu B.Cu) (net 22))
 (segment (start 132.6 100.275) (end 132.6 100.75) (width 0.25) (layer F.Cu) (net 22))
 (segment (start 132.6 100.75) (end 132.4 100.95) (width 0.25) (layer F.Cu) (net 22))
 (segment (start 132.4 100.95) (end 129.903 100.95) (width 0.25) (layer F.Cu) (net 22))
 (segment (start 129.903 100.95) (end 129.888 100.965) (width 0.25) (layer F.Cu) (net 22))
 (segment (start 129.888 100.965) (end 129.853 101) (width 0.25) (layer F.Cu) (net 22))
 (segment (start 129.853 101) (end 126.8 101) (width 0.25) (layer F.Cu) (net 22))
 (segment (start 126.8 101) (end 121.5 101) (width 0.25) (layer F.Cu) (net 22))
 (segment (start 120.8 100.3) (end 114.2 100.3) (width 0.25) (layer F.Cu) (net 22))
 (segment (start 121.5 101) (end 120.8 100.3) (width 0.25) (layer F.Cu) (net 22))
 (segment (start 114.046 100.33) (end 114.076 100.3) (width 0.25) (layer F.Cu) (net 22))
 (segment (start 129.823 100.9) (end 129.888 100.965) (width 0.25) (layer F.Cu) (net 22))
 (segment (start 132.825 101.6) (end 132.829804 101.595196) (width 0.25) (layer F.Cu) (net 23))
 (segment (start 132.829804 101.595196) (end 132.825 101.6) (width 0.25) (layer F.Cu) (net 23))
 (segment (start 132.825 101.6) (end 132.825 101.35) (width 0.25) (layer F.Cu) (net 23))
 (segment (start 132.85 101.325) (end 132.825 101.35) (width 0.25) (layer F.Cu) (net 23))
 (segment (start 132.825 101.35) (end 133.6 100.575) (width 0.25) (layer F.Cu) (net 23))
 (segment (start 134.6 101.6) (end 132.825 101.6) (width 0.25) (layer B.Cu) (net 23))
 (via (at 132.825 101.6) (size 0.6) (drill 0.4) (layers F.Cu B.Cu) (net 23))
 (segment (start 133.6 100.575) (end 133.6 99.475) (width 0.25) (layer F.Cu) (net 23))
 (segment (start 133.6 99.475) (end 133.025 98.9) (width 0.25) (layer F.Cu) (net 23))
 (segment (start 133.025 98.9) (end 130.025 98.9) (width 0.25) (layer F.Cu) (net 23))
 (segment (start 130.025 98.9) (end 129.9 99.025) (width 0.25) (layer F.Cu) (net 23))
 (segment (start 129.9 99.025) (end 129.9 99.683) (width 0.25) (layer F.Cu) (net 23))
 (segment (start 129.9 99.683) (end 129.888 99.695) (width 0.25) (layer F.Cu) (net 23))
 (segment (start 134.6 102.9) (end 134.6 101.6) (width 0.3048) (layer B.Cu) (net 23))
 (segment (start 134.6 101.6) (end 134.6 100.3) (width 0.3048) (layer B.Cu) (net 23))
 (segment (start 138.6 103.5) (end 138.595 103.505) (width 0.3048) (layer F.Cu) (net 24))
 (segment (start 139.5 102.5) (end 139.5 102.6) (width 0.3048) (layer F.Cu) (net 24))
 (segment (start 139.5 102.6) (end 138.6 103.5) (width 0.3048) (layer F.Cu) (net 24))
 (segment (start 143.286 100.3) (end 140.2 100.3) (width 0.3048) (layer F.Cu) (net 24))
 (segment (start 140.2 100.3) (end 139.5 101) (width 0.3048) (layer F.Cu) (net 24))
 (segment (start 139.5 101) (end 139.5 102.5) (width 0.3048) (layer F.Cu) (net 24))
 (segment (start 138.595 103.505) (end 135.288 103.505) (width 0.3048) (layer F.Cu) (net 24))
 (segment (start 143.51 100.076) (end 143.286 100.3) (width 0.3048) (layer F.Cu) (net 24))
 (segment (start 135.288 103.505) (end 135.5 103.5) (width 0.3048) (layer F.Cu) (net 24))
 (segment (start 139.75 97.55) (end 139.764 97.536) (width 0.3048) (layer F.Cu) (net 26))
 (segment (start 139.764 97.536) (end 143.51 97.536) (width 0.3048) (layer F.Cu) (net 26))
 (segment (start 135.288 99.695) (end 135.293 99.7) (width 0.3048) (layer F.Cu) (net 26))
 (segment (start 135.293 99.7) (end 138.5 99.7) (width 0.3048) (layer F.Cu) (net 26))
 (segment (start 138.5 99.7) (end 139.2 99) (width 0.3048) (layer F.Cu) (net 26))
 (segment (start 139.2 99) (end 139.2 98.1) (width 0.3048) (layer F.Cu) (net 26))
 (segment (start 139.2 98.1) (end 139.75 97.55) (width 0.3048) (layer F.Cu) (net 26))
 (segment (start 135.4 99.7) (end 135.367 99.7) (width 0.3048) (layer F.Cu) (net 26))
 (segment (start 143.51 110.236) (end 143.499 110.225) (width 0.25) (layer B.Cu) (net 9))
 (segment (start 143.499 110.225) (end 140.175 110.225) (width 0.25) (layer B.Cu) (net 9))
 (segment (start 140.175 110.225) (end 140.1 110.225) (width 0.25) (layer B.Cu) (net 9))
 (segment (start 140.1 110.225) (end 139.075 109.2) (width 0.25) (layer B.Cu) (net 9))
 (segment (start 139.075 109.2) (end 139.075 93.9) (width 0.25) (layer B.Cu) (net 9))
 (segment (start 139.075 93.9) (end 138.25 93.075) (width 0.25) (layer B.Cu) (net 9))
 (via (at 138.25 93.075) (size 0.6) (drill 0.4) (layers F.Cu B.Cu) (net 9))
 (segment (start 138.25 93.075) (end 135.20242 93.075) (width 0.25) (layer F.Cu) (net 9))
 (segment (start 135.20242 93.075) (end 135.18642 93.091) (width 0.25) (layer F.Cu) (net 9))
 (segment (start 143.51 107.696) (end 143.506 107.7) (width 0.25) (layer B.Cu) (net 10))
 (segment (start 143.506 107.7) (end 140.95 107.7) (width 0.25) (layer B.Cu) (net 10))
 (segment (start 140.95 107.7) (end 140.175 106.925) (width 0.25) (layer B.Cu) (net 10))
 (segment (start 140.175 106.925) (end 140.175 93.05) (width 0.25) (layer B.Cu) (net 10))
 (segment (start 140.175 93.05) (end 138.975 91.85) (width 0.25) (layer B.Cu) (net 10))
 (via (at 138.975 91.85) (size 0.6) (drill 0.4) (layers F.Cu B.Cu) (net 10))
 (segment (start 138.975 91.85) (end 135.21542 91.85) (width 0.25) (layer F.Cu) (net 10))
 (segment (start 135.21542 91.85) (end 135.18642 91.821) (width 0.25) (layer F.Cu) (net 10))
 (segment (start 139.625 90.675) (end 139.501 90.551) (width 0.25) (layer F.Cu) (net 11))
 (segment (start 139.501 90.551) (end 135.18642 90.551) (width 0.25) (layer F.Cu) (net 11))
 (segment (start 143.51 94.996) (end 143.506 95) (width 0.25) (layer F.Cu) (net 11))
 (segment (start 143.506 95) (end 141.875 95) (width 0.25) (layer F.Cu) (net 11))
 (segment (start 141.875 95) (end 141.85 95) (width 0.25) (layer F.Cu) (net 11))
 (segment (start 141.85 95) (end 141.75 95) (width 0.25) (layer F.Cu) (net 11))
 (segment (start 141.75 95) (end 141.2 94.45) (width 0.25) (layer F.Cu) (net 11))
 (segment (start 141.2 94.45) (end 141.2 92.8) (width 0.25) (layer F.Cu) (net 11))
 (segment (start 141.2 92.8) (end 140.075 91.675) (width 0.25) (layer F.Cu) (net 11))
 (segment (start 140.075 91.675) (end 140.075 91.125) (width 0.25) (layer F.Cu) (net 11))
 (segment (start 140.075 91.125) (end 139.625 90.675) (width 0.25) (layer F.Cu) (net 11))
 (segment (start 135.18642 90.551) (end 135.23742 90.5) (width 0.3048) (layer F.Cu) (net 11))
 (segment (start 143.51 92.456) (end 143.504 92.45) (width 0.25) (layer F.Cu) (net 12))
 (segment (start 143.504 92.45) (end 142.125 92.45) (width 0.25) (layer F.Cu) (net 12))
 (segment (start 142.125 92.45) (end 141.325 91.65) (width 0.25) (layer F.Cu) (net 12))
 (segment (start 141.325 91.65) (end 141.325 89.825) (width 0.25) (layer F.Cu) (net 12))
 (segment (start 141.325 89.825) (end 140.75 89.25) (width 0.25) (layer F.Cu) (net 12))
 (segment (start 140.75 89.25) (end 135.21742 89.25) (width 0.25) (layer F.Cu) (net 12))
 (segment (start 135.21742 89.25) (end 135.18642 89.281) (width 0.25) (layer F.Cu) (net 12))
 (segment (start 135.20542 89.3) (end 135.18642 89.281) (width 0.3048) (layer F.Cu) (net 12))
 (segment (start 143.51 92.456) (end 143.466 92.5) (width 0.3048) (layer F.Cu) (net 12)))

